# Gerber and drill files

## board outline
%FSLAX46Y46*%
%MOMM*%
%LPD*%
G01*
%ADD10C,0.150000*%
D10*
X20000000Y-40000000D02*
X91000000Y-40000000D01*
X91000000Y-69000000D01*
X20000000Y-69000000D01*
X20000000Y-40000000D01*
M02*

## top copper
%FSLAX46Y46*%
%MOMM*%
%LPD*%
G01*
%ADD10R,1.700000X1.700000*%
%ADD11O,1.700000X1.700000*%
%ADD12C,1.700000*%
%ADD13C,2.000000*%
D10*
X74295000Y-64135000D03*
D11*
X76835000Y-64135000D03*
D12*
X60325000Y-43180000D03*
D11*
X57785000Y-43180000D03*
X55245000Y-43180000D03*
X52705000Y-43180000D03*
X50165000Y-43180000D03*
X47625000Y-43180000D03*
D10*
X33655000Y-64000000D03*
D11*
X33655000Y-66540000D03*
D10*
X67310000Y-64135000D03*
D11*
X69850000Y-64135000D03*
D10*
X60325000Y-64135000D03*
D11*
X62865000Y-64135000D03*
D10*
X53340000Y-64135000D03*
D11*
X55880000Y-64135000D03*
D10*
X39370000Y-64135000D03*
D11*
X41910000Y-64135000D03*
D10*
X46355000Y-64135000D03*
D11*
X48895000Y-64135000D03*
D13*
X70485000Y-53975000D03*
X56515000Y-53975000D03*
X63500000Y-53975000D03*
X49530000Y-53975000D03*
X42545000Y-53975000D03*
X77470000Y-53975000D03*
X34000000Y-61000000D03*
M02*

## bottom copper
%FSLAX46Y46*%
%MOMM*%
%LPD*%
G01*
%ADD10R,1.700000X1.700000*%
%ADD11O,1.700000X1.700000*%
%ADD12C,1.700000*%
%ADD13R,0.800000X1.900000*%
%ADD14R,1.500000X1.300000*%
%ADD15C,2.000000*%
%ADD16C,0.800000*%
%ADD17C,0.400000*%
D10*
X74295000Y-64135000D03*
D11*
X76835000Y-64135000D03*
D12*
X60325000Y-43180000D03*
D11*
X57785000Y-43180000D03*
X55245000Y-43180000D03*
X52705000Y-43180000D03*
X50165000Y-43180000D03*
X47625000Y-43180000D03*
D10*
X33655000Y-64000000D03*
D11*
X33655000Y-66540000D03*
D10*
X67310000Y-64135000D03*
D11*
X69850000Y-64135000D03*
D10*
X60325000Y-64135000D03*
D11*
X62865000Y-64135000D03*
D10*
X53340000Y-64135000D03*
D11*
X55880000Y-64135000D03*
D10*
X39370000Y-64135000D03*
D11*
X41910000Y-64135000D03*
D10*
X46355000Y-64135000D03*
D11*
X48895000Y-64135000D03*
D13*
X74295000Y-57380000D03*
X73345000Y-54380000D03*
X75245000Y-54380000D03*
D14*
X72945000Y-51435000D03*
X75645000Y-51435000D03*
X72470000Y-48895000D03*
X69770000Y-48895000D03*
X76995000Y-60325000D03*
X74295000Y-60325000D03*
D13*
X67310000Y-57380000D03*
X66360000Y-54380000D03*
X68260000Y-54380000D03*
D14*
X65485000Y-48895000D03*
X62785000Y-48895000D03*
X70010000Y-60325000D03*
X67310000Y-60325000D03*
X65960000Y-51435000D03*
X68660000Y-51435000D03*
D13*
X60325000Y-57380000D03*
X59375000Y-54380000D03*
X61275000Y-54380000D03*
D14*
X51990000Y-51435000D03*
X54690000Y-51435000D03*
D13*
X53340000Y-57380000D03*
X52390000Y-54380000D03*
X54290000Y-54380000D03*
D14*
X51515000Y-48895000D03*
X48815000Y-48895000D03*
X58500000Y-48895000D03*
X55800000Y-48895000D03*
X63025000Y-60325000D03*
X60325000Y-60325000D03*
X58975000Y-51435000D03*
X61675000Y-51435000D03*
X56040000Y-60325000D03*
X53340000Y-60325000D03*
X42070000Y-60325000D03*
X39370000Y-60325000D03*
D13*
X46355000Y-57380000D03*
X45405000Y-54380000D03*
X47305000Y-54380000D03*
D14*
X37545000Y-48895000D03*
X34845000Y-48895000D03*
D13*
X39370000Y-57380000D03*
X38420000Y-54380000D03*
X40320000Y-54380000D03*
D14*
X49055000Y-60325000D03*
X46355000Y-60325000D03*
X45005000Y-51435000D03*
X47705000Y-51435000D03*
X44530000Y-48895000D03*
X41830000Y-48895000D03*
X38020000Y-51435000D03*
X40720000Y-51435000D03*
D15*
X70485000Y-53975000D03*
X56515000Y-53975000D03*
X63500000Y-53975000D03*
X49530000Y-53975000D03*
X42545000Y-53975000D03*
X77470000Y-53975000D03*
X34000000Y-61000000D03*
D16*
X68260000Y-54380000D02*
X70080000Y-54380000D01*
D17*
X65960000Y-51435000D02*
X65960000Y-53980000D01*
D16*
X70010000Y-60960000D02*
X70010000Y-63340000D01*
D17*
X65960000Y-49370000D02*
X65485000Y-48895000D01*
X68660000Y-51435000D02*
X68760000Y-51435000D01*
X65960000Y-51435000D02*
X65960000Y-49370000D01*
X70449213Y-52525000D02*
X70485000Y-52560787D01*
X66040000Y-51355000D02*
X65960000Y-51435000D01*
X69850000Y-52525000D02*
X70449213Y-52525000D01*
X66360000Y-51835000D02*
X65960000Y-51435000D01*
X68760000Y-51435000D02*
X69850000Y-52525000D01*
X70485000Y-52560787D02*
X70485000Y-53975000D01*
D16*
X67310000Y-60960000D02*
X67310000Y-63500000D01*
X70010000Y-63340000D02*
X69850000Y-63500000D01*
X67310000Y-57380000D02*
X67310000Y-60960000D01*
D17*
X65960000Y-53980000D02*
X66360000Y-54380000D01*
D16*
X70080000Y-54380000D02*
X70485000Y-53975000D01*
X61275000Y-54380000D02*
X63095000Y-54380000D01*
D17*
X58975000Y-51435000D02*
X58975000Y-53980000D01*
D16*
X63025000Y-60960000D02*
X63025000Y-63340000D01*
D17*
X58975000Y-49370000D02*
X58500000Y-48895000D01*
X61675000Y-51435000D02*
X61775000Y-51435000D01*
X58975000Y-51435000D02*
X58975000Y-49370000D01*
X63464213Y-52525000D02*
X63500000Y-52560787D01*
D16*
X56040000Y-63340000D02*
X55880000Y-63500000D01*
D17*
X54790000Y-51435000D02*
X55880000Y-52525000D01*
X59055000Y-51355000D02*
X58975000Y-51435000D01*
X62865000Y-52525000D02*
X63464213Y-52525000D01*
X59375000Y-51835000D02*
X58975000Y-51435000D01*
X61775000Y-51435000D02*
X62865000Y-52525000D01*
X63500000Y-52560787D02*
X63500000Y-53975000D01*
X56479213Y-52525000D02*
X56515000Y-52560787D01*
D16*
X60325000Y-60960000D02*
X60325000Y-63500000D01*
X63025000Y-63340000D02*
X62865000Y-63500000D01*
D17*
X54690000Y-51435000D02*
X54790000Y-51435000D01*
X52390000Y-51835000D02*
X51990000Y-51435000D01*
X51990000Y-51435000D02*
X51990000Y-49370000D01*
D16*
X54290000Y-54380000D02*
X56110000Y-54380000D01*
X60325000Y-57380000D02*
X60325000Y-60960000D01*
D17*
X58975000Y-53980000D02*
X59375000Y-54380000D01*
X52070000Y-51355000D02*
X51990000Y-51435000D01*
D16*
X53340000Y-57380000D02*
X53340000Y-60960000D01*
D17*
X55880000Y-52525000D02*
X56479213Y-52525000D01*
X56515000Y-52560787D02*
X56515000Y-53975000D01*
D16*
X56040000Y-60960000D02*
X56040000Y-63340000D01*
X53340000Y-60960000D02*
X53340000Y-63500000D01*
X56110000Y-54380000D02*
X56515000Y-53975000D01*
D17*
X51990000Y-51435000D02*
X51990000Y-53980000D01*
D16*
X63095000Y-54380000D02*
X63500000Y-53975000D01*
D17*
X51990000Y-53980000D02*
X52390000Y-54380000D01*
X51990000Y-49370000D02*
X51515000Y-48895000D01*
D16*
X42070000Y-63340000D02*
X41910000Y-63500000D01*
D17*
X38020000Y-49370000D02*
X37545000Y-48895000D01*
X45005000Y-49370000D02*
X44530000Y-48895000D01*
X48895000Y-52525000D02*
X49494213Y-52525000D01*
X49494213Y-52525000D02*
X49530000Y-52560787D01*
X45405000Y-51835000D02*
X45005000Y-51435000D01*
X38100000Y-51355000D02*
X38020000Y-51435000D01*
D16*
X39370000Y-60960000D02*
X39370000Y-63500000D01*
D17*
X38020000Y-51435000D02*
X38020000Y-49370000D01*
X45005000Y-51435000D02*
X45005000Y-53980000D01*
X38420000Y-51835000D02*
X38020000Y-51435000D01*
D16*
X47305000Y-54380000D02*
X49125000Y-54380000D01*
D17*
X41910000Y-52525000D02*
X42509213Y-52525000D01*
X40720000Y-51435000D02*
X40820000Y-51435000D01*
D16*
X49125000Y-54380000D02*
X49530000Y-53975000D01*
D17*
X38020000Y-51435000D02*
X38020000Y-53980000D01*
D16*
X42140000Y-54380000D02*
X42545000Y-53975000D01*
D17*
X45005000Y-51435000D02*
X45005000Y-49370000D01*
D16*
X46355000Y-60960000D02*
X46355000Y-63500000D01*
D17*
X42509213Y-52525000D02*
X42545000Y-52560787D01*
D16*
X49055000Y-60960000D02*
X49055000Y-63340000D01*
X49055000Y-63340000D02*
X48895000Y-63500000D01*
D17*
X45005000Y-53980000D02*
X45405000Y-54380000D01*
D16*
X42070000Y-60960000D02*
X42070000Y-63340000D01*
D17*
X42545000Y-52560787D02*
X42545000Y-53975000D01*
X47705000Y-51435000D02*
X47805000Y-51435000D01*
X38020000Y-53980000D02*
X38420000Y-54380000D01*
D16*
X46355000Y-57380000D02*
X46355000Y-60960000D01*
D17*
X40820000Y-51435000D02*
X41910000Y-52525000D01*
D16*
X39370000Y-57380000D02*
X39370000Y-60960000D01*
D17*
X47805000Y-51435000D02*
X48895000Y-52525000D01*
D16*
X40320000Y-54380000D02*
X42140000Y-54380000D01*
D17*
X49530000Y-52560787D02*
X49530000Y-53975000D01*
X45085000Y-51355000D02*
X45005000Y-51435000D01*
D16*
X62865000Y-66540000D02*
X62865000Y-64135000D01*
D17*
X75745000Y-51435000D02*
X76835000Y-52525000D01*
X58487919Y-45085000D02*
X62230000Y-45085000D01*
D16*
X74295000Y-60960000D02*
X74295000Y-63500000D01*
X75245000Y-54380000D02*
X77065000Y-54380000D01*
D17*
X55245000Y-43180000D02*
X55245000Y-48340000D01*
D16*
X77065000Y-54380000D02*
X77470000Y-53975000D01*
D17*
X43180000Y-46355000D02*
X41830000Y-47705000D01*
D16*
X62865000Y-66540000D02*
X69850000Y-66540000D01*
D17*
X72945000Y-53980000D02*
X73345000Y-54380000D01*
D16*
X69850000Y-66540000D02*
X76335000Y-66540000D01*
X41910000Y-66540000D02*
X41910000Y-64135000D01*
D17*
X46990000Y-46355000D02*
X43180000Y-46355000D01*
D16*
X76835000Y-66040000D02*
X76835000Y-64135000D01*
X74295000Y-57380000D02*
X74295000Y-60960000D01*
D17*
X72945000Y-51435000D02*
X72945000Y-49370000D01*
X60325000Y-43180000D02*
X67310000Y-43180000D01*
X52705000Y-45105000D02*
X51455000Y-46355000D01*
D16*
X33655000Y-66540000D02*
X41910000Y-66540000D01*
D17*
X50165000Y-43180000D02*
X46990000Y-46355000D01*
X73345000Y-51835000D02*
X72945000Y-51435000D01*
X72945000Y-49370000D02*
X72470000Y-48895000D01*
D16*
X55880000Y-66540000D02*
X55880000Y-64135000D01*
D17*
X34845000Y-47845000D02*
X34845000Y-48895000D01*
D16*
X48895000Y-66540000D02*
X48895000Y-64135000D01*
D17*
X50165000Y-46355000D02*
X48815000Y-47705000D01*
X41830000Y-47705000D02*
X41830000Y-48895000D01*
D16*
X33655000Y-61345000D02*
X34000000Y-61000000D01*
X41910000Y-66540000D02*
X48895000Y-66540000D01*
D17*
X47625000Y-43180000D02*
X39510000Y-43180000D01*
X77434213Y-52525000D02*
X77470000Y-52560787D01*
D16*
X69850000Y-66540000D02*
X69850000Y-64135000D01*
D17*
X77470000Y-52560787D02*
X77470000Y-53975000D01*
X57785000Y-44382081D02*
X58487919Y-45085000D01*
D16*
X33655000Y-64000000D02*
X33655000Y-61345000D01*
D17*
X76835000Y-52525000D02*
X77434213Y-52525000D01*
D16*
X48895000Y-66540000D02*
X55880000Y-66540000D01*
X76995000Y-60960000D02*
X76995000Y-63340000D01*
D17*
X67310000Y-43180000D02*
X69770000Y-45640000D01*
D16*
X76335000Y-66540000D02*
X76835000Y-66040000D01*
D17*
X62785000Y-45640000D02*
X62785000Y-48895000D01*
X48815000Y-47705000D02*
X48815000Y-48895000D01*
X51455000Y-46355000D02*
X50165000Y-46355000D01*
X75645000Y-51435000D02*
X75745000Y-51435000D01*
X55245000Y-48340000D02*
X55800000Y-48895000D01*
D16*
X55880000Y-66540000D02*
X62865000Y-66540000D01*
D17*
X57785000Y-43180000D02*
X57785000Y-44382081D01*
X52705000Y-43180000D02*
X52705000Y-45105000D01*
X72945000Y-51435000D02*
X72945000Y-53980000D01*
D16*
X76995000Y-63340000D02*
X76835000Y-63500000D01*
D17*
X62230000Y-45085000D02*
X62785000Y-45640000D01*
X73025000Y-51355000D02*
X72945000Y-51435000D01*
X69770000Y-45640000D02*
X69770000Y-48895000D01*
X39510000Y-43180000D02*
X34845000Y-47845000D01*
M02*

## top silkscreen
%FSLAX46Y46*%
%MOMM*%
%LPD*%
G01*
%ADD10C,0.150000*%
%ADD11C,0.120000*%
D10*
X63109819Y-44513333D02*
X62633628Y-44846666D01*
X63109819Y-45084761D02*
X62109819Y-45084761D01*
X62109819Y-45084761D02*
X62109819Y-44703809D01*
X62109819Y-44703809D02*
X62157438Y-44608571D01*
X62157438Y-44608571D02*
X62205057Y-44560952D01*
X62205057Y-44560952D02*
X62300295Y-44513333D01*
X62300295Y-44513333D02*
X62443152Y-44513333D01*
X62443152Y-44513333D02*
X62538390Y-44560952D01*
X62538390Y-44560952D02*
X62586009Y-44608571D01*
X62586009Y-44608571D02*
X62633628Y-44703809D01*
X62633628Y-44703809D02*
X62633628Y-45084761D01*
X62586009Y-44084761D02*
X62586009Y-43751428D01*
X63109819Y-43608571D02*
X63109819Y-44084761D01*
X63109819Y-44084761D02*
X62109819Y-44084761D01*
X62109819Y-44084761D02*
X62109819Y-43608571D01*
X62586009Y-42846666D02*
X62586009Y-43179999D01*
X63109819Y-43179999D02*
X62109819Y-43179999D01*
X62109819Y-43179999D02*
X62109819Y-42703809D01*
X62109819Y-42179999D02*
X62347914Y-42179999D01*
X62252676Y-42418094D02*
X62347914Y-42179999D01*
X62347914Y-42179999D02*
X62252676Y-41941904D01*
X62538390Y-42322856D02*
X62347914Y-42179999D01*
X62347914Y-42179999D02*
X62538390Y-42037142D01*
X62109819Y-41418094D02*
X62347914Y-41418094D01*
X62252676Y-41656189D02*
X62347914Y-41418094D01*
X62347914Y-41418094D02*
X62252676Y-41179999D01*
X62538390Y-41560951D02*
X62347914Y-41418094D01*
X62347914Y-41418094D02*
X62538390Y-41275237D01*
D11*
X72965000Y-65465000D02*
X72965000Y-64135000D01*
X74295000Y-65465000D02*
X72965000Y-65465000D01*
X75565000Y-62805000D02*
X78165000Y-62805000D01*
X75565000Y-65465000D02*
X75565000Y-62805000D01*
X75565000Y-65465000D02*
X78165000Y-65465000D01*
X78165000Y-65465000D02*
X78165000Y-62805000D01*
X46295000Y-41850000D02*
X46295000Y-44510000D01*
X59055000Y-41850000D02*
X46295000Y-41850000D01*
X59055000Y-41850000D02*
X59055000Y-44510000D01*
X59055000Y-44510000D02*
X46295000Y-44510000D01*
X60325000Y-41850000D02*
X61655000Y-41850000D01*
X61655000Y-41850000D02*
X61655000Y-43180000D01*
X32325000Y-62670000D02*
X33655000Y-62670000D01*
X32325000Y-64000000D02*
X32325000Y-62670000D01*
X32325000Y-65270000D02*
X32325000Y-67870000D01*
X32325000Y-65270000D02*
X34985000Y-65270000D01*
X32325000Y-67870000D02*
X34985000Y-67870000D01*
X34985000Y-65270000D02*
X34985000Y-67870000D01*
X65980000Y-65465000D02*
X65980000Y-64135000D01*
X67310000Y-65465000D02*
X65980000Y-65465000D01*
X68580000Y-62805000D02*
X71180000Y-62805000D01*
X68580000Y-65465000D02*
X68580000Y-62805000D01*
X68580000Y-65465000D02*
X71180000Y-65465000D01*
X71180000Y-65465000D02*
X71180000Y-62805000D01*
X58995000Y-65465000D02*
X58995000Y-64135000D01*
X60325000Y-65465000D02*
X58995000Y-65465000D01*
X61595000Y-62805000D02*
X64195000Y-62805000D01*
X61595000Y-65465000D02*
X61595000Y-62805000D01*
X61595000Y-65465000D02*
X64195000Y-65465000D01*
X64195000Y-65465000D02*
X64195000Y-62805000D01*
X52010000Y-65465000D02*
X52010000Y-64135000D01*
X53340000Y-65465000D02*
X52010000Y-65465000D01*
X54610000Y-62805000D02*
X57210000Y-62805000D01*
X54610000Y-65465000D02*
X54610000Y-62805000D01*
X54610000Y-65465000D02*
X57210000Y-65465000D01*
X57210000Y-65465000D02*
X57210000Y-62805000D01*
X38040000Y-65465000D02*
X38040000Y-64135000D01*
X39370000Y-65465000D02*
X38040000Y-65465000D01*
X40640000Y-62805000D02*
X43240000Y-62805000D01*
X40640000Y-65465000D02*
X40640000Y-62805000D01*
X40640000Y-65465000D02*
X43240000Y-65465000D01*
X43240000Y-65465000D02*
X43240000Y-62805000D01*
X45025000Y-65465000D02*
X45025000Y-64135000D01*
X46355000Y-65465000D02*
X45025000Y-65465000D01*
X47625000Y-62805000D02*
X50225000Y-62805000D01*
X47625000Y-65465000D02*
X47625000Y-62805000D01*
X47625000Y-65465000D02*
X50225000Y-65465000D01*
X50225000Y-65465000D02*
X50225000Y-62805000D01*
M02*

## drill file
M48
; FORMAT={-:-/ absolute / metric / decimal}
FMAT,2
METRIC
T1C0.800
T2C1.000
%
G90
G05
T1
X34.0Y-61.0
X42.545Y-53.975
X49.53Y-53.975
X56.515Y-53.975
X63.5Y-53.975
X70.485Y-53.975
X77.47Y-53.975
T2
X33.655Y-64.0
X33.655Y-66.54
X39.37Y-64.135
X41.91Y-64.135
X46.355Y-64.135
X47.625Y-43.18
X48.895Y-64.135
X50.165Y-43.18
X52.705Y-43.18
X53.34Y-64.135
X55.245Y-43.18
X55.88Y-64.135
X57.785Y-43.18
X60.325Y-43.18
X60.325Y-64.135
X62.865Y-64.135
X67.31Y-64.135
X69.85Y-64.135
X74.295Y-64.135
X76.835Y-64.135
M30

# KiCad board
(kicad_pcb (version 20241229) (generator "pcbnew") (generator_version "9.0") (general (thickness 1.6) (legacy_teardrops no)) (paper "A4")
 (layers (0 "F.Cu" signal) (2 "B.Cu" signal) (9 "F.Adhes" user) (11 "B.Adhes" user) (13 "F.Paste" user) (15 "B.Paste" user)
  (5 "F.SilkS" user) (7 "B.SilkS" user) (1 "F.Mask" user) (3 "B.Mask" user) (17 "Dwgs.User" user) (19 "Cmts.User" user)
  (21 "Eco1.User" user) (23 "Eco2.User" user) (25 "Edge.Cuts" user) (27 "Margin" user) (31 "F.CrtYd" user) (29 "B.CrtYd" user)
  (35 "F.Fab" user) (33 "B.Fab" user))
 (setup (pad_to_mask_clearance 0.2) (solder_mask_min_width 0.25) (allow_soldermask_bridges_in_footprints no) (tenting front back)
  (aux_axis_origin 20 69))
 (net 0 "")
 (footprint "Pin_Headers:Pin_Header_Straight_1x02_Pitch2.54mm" (layer "F.Cu") (at 74.295 64.135 90)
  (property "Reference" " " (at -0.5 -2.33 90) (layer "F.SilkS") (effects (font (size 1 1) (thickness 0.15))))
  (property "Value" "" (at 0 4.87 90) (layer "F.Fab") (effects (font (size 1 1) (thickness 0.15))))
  (fp_line (start -1.33 -1.33) (end 0 -1.33) (stroke (width 0.12) (type solid)) (layer "F.SilkS"))
  (fp_line (start -1.33 0) (end -1.33 -1.33) (stroke (width 0.12) (type solid)) (layer "F.SilkS"))
  (fp_line (start 1.33 1.27) (end 1.33 3.87) (stroke (width 0.12) (type solid)) (layer "F.SilkS"))
  (fp_line (start -1.33 1.27) (end 1.33 1.27) (stroke (width 0.12) (type solid)) (layer "F.SilkS"))
  (fp_line (start -1.33 1.27) (end -1.33 3.87) (stroke (width 0.12) (type solid)) (layer "F.SilkS"))
  (fp_line (start -1.33 3.87) (end 1.33 3.87) (stroke (width 0.12) (type solid)) (layer "F.SilkS"))
  (pad "1" thru_hole rect (at 0 0 90) (size 1.7 1.7) (drill 1) (layers "*.Cu" "*.Mask") (remove_unused_layers no))
  (pad "2" thru_hole oval (at 0 2.54 90) (size 1.7 1.7) (drill 1) (layers "*.Cu" "*.Mask") (remove_unused_layers no)))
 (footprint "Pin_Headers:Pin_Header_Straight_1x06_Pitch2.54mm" (layer "F.Cu") (at 60.325 43.18 -90)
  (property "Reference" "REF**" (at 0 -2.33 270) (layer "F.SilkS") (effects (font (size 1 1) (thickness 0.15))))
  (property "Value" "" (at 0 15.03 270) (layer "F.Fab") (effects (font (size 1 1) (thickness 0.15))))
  (fp_line (start -1.33 14.03) (end 1.33 14.03) (stroke (width 0.12) (type solid)) (layer "F.SilkS"))
  (fp_line (start -1.33 1.27) (end -1.33 14.03) (stroke (width 0.12) (type solid)) (layer "F.SilkS"))
  (fp_line (start -1.33 1.27) (end 1.33 1.27) (stroke (width 0.12) (type solid)) (layer "F.SilkS"))
  (fp_line (start 1.33 1.27) (end 1.33 14.03) (stroke (width 0.12) (type solid)) (layer "F.SilkS"))
  (fp_line (start -1.33 0) (end -1.33 -1.33) (stroke (width 0.12) (type solid)) (layer "F.SilkS"))
  (fp_line (start -1.33 -1.33) (end 0 -1.33) (stroke (width 0.12) (type solid)) (layer "F.SilkS"))
  (pad "1" thru_hole circle (at 0 0 270) (size 1.7 1.7) (drill 1) (layers "*.Cu" "*.Mask") (remove_unused_layers no))
  (pad "2" thru_hole oval (at 0 2.54 270) (size 1.7 1.7) (drill 1) (layers "*.Cu" "*.Mask") (remove_unused_layers no))
  (pad "3" thru_hole oval (at 0 5.08 270) (size 1.7 1.7) (drill 1) (layers "*.Cu" "*.Mask") (remove_unused_layers no))
  (pad "4" thru_hole oval (at 0 7.62 270) (size 1.7 1.7) (drill 1) (layers "*.Cu" "*.Mask") (remove_unused_layers no))
  (pad "5" thru_hole oval (at 0 10.16 270) (size 1.7 1.7) (drill 1) (layers "*.Cu" "*.Mask") (remove_unused_layers no))
  (pad "6" thru_hole oval (at 0 12.7 270) (size 1.7 1.7) (drill 1) (layers "*.Cu" "*.Mask") (remove_unused_layers no)))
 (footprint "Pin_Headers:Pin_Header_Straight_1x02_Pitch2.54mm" (layer "F.Cu") (at 33.655 64)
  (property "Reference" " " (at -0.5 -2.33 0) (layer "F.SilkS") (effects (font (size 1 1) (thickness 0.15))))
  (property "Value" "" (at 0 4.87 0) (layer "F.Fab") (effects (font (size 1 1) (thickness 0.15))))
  (fp_line (start -1.33 -1.33) (end 0 -1.33) (stroke (width 0.12) (type solid)) (layer "F.SilkS"))
  (fp_line (start -1.33 0) (end -1.33 -1.33) (stroke (width 0.12) (type solid)) (layer "F.SilkS"))
  (fp_line (start -1.33 1.27) (end -1.33 3.87) (stroke (width 0.12) (type solid)) (layer "F.SilkS"))
  (fp_line (start -1.33 1.27) (end 1.33 1.27) (stroke (width 0.12) (type solid)) (layer "F.SilkS"))
  (fp_line (start -1.33 3.87) (end 1.33 3.87) (stroke (width 0.12) (type solid)) (layer "F.SilkS"))
  (fp_line (start 1.33 1.27) (end 1.33 3.87) (stroke (width 0.12) (type solid)) (layer "F.SilkS"))
  (pad "1" thru_hole rect (at 0 0) (size 1.7 1.7) (drill 1) (layers "*.Cu" "*.Mask") (remove_unused_layers no))
  (pad "2" thru_hole oval (at 0 2.54) (size 1.7 1.7) (drill 1) (layers "*.Cu" "*.Mask") (remove_unused_layers no)))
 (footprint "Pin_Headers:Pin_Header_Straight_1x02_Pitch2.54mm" (layer "F.Cu") (at 67.31 64.135 90)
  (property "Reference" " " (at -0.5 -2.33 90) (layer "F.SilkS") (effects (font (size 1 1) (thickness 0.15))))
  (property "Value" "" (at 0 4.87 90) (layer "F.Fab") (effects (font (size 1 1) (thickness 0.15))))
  (fp_line (start -1.33 -1.33) (end 0 -1.33) (stroke (width 0.12) (type solid)) (layer "F.SilkS"))
  (fp_line (start -1.33 0) (end -1.33 -1.33) (stroke (width 0.12) (type solid)) (layer "F.SilkS"))
  (fp_line (start 1.33 1.27) (end 1.33 3.87) (stroke (width 0.12) (type solid)) (layer "F.SilkS"))
  (fp_line (start -1.33 1.27) (end 1.33 1.27) (stroke (width 0.12) (type solid)) (layer "F.SilkS"))
  (fp_line (start -1.33 1.27) (end -1.33 3.87) (stroke (width 0.12) (type solid)) (layer "F.SilkS"))
  (fp_line (start -1.33 3.87) (end 1.33 3.87) (stroke (width 0.12) (type solid)) (layer "F.SilkS"))
  (pad "1" thru_hole rect (at 0 0 90) (size 1.7 1.7) (drill 1) (layers "*.Cu" "*.Mask") (remove_unused_layers no))
  (pad "2" thru_hole oval (at 0 2.54 90) (size 1.7 1.7) (drill 1) (layers "*.Cu" "*.Mask") (remove_unused_layers no)))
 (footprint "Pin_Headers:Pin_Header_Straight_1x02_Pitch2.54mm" (layer "F.Cu") (at 60.325 64.135 90)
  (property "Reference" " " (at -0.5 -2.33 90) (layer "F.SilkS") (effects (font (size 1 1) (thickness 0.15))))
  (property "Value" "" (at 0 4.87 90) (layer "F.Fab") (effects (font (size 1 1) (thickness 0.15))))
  (fp_line (start -1.33 -1.33) (end 0 -1.33) (stroke (width 0.12) (type solid)) (layer "F.SilkS"))
  (fp_line (start -1.33 0) (end -1.33 -1.33) (stroke (width 0.12) (type solid)) (layer "F.SilkS"))
  (fp_line (start 1.33 1.27) (end 1.33 3.87) (stroke (width 0.12) (type solid)) (layer "F.SilkS"))
  (fp_line (start -1.33 1.27) (end 1.33 1.27) (stroke (width 0.12) (type solid)) (layer "F.SilkS"))
  (fp_line (start -1.33 1.27) (end -1.33 3.87) (stroke (width 0.12) (type solid)) (layer "F.SilkS"))
  (fp_line (start -1.33 3.87) (end 1.33 3.87) (stroke (width 0.12) (type solid)) (layer "F.SilkS"))
  (pad "1" thru_hole rect (at 0 0 90) (size 1.7 1.7) (drill 1) (layers "*.Cu" "*.Mask") (remove_unused_layers no))
  (pad "2" thru_hole oval (at 0 2.54 90) (size 1.7 1.7) (drill 1) (layers "*.Cu" "*.Mask") (remove_unused_layers no)))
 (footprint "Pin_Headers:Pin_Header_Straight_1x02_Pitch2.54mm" (layer "F.Cu") (at 53.34 64.135 90)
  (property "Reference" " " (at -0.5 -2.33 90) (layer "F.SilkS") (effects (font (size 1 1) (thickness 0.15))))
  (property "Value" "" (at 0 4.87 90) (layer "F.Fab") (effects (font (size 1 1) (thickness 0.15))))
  (fp_line (start -1.33 -1.33) (end 0 -1.33) (stroke (width 0.12) (type solid)) (layer "F.SilkS"))
  (fp_line (start -1.33 0) (end -1.33 -1.33) (stroke (width 0.12) (type solid)) (layer "F.SilkS"))
  (fp_line (start 1.33 1.27) (end 1.33 3.87) (stroke (width 0.12) (type solid)) (layer "F.SilkS"))
  (fp_line (start -1.33 1.27) (end 1.33 1.27) (stroke (width 0.12) (type solid)) (layer "F.SilkS"))
  (fp_line (start -1.33 1.27) (end -1.33 3.87) (stroke (width 0.12) (type solid)) (layer "F.SilkS"))
  (fp_line (start -1.33 3.87) (end 1.33 3.87) (stroke (width 0.12) (type solid)) (layer "F.SilkS"))
  (pad "1" thru_hole rect (at 0 0 90) (size 1.7 1.7) (drill 1) (layers "*.Cu" "*.Mask") (remove_unused_layers no))
  (pad "2" thru_hole oval (at 0 2.54 90) (size 1.7 1.7) (drill 1) (layers "*.Cu" "*.Mask") (remove_unused_layers no)))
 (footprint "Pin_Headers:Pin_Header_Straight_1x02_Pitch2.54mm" (layer "F.Cu") (at 39.37 64.135 90)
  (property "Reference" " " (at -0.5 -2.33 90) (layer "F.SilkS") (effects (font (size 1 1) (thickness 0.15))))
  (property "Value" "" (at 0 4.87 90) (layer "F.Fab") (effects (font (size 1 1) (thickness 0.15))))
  (fp_line (start -1.33 -1.33) (end 0 -1.33) (stroke (width 0.12) (type solid)) (layer "F.SilkS"))
  (fp_line (start -1.33 0) (end -1.33 -1.33) (stroke (width 0.12) (type solid)) (layer "F.SilkS"))
  (fp_line (start 1.33 1.27) (end 1.33 3.87) (stroke (width 0.12) (type solid)) (layer "F.SilkS"))
  (fp_line (start -1.33 1.27) (end 1.33 1.27) (stroke (width 0.12) (type solid)) (layer "F.SilkS"))
  (fp_line (start -1.33 1.27) (end -1.33 3.87) (stroke (width 0.12) (type solid)) (layer "F.SilkS"))
  (fp_line (start -1.33 3.87) (end 1.33 3.87) (stroke (width 0.12) (type solid)) (layer "F.SilkS"))
  (pad "1" thru_hole rect (at 0 0 90) (size 1.7 1.7) (drill 1) (layers "*.Cu" "*.Mask") (remove_unused_layers no))
  (pad "2" thru_hole oval (at 0 2.54 90) (size 1.7 1.7) (drill 1) (layers "*.Cu" "*.Mask") (remove_unused_layers no)))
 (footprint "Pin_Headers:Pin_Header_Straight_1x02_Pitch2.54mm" (layer "F.Cu") (at 46.355 64.135 90)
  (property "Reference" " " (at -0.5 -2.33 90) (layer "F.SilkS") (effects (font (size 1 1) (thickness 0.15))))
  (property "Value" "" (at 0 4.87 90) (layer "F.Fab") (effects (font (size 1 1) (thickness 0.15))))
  (fp_line (start -1.33 -1.33) (end 0 -1.33) (stroke (width 0.12) (type solid)) (layer "F.SilkS"))
  (fp_line (start -1.33 0) (end -1.33 -1.33) (stroke (width 0.12) (type solid)) (layer "F.SilkS"))
  (fp_line (start 1.33 1.27) (end 1.33 3.87) (stroke (width 0.12) (type solid)) (layer "F.SilkS"))
  (fp_line (start -1.33 1.27) (end 1.33 1.27) (stroke (width 0.12) (type solid)) (layer "F.SilkS"))
  (fp_line (start -1.33 1.27) (end -1.33 3.87) (stroke (width 0.12) (type solid)) (layer "F.SilkS"))
  (fp_line (start -1.33 3.87) (end 1.33 3.87) (stroke (width 0.12) (type solid)) (layer "F.SilkS"))
  (pad "1" thru_hole rect (at 0 0 90) (size 1.7 1.7) (drill 1) (layers "*.Cu" "*.Mask") (remove_unused_layers no))
  (pad "2" thru_hole oval (at 0 2.54 90) (size 1.7 1.7) (drill 1) (layers "*.Cu" "*.Mask") (remove_unused_layers no)))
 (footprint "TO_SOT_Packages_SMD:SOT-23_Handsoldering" (layer "B.Cu") (at 74.295 55.88 -90)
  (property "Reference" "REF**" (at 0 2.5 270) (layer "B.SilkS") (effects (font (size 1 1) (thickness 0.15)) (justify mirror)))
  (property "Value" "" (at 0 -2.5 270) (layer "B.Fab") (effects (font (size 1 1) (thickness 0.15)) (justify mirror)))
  (pad "D" smd rect (at 1.5 0 270) (size 1.9 0.8) (layers "B.Cu" "B.Mask" "B.Paste"))
  (pad "G" smd rect (at -1.5 0.95 270) (size 1.9 0.8) (layers "B.Cu" "B.Mask" "B.Paste"))
  (pad "S" smd rect (at -1.5 -0.95 270) (size 1.9 0.8) (layers "B.Cu" "B.Mask" "B.Paste")))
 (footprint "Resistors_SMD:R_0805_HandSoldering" (layer "B.Cu") (at 74.295 51.435)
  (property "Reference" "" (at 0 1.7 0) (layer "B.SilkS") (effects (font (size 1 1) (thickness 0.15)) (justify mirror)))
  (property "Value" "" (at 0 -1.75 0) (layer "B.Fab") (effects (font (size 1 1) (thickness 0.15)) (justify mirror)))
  (pad "1" smd rect (at -1.35 0) (size 1.5 1.3) (layers "B.Cu" "B.Mask" "B.Paste"))
  (pad "2" smd rect (at 1.35 0) (size 1.5 1.3) (layers "B.Cu" "B.Mask" "B.Paste")))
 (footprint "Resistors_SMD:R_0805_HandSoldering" (layer "B.Cu") (at 71.12 48.895 180)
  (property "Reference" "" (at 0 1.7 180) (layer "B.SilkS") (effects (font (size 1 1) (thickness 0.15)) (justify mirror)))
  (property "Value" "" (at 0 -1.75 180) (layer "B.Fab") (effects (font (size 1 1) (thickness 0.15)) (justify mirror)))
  (pad "1" smd rect (at -1.35 0 180) (size 1.5 1.3) (layers "B.Cu" "B.Mask" "B.Paste"))
  (pad "2" smd rect (at 1.35 0 180) (size 1.5 1.3) (layers "B.Cu" "B.Mask" "B.Paste")))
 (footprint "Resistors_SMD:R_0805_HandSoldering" (layer "B.Cu") (at 75.645 60.325 180)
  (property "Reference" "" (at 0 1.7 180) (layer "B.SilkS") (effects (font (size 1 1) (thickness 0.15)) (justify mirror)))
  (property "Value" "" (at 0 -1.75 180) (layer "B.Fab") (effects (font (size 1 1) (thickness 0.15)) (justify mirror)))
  (pad "1" smd rect (at -1.35 0 180) (size 1.5 1.3) (layers "B.Cu" "B.Mask" "B.Paste"))
  (pad "2" smd rect (at 1.35 0 180) (size 1.5 1.3) (layers "B.Cu" "B.Mask" "B.Paste")))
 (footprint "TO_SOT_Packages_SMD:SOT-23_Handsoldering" (layer "B.Cu") (at 67.31 55.88 -90)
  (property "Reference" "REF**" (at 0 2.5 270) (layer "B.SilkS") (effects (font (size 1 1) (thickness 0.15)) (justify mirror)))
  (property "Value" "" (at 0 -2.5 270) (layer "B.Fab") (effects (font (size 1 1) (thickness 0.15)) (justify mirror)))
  (pad "D" smd rect (at 1.5 0 270) (size 1.9 0.8) (layers "B.Cu" "B.Mask" "B.Paste"))
  (pad "G" smd rect (at -1.5 0.95 270) (size 1.9 0.8) (layers "B.Cu" "B.Mask" "B.Paste"))
  (pad "S" smd rect (at -1.5 -0.95 270) (size 1.9 0.8) (layers "B.Cu" "B.Mask" "B.Paste")))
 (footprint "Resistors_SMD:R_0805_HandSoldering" (layer "B.Cu") (at 64.135 48.895 180)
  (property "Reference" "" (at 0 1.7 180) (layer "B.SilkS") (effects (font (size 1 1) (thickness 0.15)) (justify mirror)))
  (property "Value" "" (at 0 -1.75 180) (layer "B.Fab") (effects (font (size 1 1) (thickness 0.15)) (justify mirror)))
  (pad "1" smd rect (at -1.35 0 180) (size 1.5 1.3) (layers "B.Cu" "B.Mask" "B.Paste"))
  (pad "2" smd rect (at 1.35 0 180) (size 1.5 1.3) (layers "B.Cu" "B.Mask" "B.Paste")))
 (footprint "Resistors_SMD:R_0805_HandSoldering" (layer "B.Cu") (at 68.66 60.325 180)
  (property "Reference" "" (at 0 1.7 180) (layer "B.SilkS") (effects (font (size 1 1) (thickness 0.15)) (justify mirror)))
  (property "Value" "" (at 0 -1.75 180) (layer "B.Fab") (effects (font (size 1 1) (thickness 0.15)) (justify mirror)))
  (pad "1" smd rect (at -1.35 0 180) (size 1.5 1.3) (layers "B.Cu" "B.Mask" "B.Paste"))
  (pad "2" smd rect (at 1.35 0 180) (size 1.5 1.3) (layers "B.Cu" "B.Mask" "B.Paste")))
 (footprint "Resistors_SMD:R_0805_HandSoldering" (layer "B.Cu") (at 67.31 51.435)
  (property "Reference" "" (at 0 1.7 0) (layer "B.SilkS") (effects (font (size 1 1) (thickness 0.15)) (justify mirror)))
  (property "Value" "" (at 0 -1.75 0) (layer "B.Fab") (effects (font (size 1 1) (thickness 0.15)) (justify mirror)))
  (pad "1" smd rect (at -1.35 0) (size 1.5 1.3) (layers "B.Cu" "B.Mask" "B.Paste"))
  (pad "2" smd rect (at 1.35 0) (size 1.5 1.3) (layers "B.Cu" "B.Mask" "B.Paste")))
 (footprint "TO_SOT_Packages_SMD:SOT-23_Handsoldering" (layer "B.Cu") (at 60.325 55.88 -90)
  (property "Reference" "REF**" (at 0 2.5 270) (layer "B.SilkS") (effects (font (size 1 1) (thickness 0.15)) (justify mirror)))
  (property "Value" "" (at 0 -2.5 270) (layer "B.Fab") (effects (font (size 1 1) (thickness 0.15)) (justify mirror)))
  (pad "D" smd rect (at 1.5 0 270) (size 1.9 0.8) (layers "B.Cu" "B.Mask" "B.Paste"))
  (pad "G" smd rect (at -1.5 0.95 270) (size 1.9 0.8) (layers "B.Cu" "B.Mask" "B.Paste"))
  (pad "S" smd rect (at -1.5 -0.95 270) (size 1.9 0.8) (layers "B.Cu" "B.Mask" "B.Paste")))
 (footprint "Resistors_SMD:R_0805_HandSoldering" (layer "B.Cu") (at 53.34 51.435)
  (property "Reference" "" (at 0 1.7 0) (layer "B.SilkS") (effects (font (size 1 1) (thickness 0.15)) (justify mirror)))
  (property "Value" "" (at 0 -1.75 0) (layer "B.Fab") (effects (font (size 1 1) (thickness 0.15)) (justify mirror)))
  (pad "1" smd rect (at -1.35 0) (size 1.5 1.3) (layers "B.Cu" "B.Mask" "B.Paste"))
  (pad "2" smd rect (at 1.35 0) (size 1.5 1.3) (layers "B.Cu" "B.Mask" "B.Paste")))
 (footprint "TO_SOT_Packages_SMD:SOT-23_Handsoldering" (layer "B.Cu") (at 53.34 55.88 -90)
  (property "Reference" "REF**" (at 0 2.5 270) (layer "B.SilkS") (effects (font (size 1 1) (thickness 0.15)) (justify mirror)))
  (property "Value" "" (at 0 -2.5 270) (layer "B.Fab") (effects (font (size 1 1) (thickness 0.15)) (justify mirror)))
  (pad "D" smd rect (at 1.5 0 270) (size 1.9 0.8) (layers "B.Cu" "B.Mask" "B.Paste"))
  (pad "G" smd rect (at -1.5 0.95 270) (size 1.9 0.8) (layers "B.Cu" "B.Mask" "B.Paste"))
  (pad "S" smd rect (at -1.5 -0.95 270) (size 1.9 0.8) (layers "B.Cu" "B.Mask" "B.Paste")))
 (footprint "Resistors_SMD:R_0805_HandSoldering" (layer "B.Cu") (at 50.165 48.895 180)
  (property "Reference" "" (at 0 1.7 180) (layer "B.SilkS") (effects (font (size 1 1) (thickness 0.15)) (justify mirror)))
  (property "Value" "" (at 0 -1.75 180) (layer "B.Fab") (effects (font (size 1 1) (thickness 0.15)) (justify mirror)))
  (pad "1" smd rect (at -1.35 0 180) (size 1.5 1.3) (layers "B.Cu" "B.Mask" "B.Paste"))
  (pad "2" smd rect (at 1.35 0 180) (size 1.5 1.3) (layers "B.Cu" "B.Mask" "B.Paste")))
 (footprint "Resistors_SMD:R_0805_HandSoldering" (layer "B.Cu") (at 57.15 48.895 180)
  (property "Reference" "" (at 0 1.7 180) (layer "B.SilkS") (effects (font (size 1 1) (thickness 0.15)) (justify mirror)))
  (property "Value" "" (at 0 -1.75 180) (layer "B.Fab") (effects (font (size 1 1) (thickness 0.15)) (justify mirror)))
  (pad "1" smd rect (at -1.35 0 180) (size 1.5 1.3) (layers "B.Cu" "B.Mask" "B.Paste"))
  (pad "2" smd rect (at 1.35 0 180) (size 1.5 1.3) (layers "B.Cu" "B.Mask" "B.Paste")))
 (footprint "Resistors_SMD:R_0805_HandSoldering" (layer "B.Cu") (at 61.675 60.325 180)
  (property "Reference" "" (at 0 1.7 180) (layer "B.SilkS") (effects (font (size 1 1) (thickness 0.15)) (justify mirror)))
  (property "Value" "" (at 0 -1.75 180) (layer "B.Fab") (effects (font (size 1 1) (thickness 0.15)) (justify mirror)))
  (pad "1" smd rect (at -1.35 0 180) (size 1.5 1.3) (layers "B.Cu" "B.Mask" "B.Paste"))
  (pad "2" smd rect (at 1.35 0 180) (size 1.5 1.3) (layers "B.Cu" "B.Mask" "B.Paste")))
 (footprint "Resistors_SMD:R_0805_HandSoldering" (layer "B.Cu") (at 60.325 51.435)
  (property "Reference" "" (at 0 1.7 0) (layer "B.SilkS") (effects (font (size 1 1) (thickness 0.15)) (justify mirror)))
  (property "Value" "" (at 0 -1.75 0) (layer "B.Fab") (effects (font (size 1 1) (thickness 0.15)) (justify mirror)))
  (pad "1" smd rect (at -1.35 0) (size 1.5 1.3) (layers "B.Cu" "B.Mask" "B.Paste"))
  (pad "2" smd rect (at 1.35 0) (size 1.5 1.3) (layers "B.Cu" "B.Mask" "B.Paste")))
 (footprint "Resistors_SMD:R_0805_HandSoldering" (layer "B.Cu") (at 54.69 60.325 180)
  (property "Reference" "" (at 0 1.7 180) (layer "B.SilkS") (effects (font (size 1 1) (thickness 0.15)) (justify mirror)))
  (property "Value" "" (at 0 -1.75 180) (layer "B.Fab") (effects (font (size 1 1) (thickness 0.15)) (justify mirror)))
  (pad "1" smd rect (at -1.35 0 180) (size 1.5 1.3) (layers "B.Cu" "B.Mask" "B.Paste"))
  (pad "2" smd rect (at 1.35 0 180) (size 1.5 1.3) (layers "B.Cu" "B.Mask" "B.Paste")))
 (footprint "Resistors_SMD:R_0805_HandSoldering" (layer "B.Cu") (at 40.72 60.325 180)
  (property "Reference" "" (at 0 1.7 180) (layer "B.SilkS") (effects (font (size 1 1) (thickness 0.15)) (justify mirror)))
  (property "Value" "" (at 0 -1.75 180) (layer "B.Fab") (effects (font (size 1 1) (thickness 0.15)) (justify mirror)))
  (pad "1" smd rect (at -1.35 0 180) (size 1.5 1.3) (layers "B.Cu" "B.Mask" "B.Paste"))
  (pad "2" smd rect (at 1.35 0 180) (size 1.5 1.3) (layers "B.Cu" "B.Mask" "B.Paste")))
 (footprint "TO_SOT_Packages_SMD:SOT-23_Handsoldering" (layer "B.Cu") (at 46.355 55.88 -90)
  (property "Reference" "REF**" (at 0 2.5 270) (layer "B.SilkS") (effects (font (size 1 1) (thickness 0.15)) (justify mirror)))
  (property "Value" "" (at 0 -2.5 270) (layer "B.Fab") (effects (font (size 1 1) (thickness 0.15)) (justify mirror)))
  (pad "D" smd rect (at 1.5 0 270) (size 1.9 0.8) (layers "B.Cu" "B.Mask" "B.Paste"))
  (pad "G" smd rect (at -1.5 0.95 270) (size 1.9 0.8) (layers "B.Cu" "B.Mask" "B.Paste"))
  (pad "S" smd rect (at -1.5 -0.95 270) (size 1.9 0.8) (layers "B.Cu" "B.Mask" "B.Paste")))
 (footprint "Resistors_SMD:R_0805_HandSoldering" (layer "B.Cu") (at 36.195 48.895 180)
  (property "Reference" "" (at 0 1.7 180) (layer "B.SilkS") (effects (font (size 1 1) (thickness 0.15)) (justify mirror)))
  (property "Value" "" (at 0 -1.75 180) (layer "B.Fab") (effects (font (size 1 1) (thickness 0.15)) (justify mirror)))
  (pad "1" smd rect (at -1.35 0 180) (size 1.5 1.3) (layers "B.Cu" "B.Mask" "B.Paste"))
  (pad "2" smd rect (at 1.35 0 180) (size 1.5 1.3) (layers "B.Cu" "B.Mask" "B.Paste")))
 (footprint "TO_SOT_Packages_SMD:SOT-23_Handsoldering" (layer "B.Cu") (at 39.37 55.88 -90)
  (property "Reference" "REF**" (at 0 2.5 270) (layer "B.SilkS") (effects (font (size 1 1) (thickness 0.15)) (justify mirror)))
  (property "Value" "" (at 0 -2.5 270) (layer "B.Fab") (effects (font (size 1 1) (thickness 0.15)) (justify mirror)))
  (pad "D" smd rect (at 1.5 0 270) (size 1.9 0.8) (layers "B.Cu" "B.Mask" "B.Paste"))
  (pad "G" smd rect (at -1.5 0.95 270) (size 1.9 0.8) (layers "B.Cu" "B.Mask" "B.Paste"))
  (pad "S" smd rect (at -1.5 -0.95 270) (size 1.9 0.8) (layers "B.Cu" "B.Mask" "B.Paste")))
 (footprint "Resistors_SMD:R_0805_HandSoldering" (layer "B.Cu") (at 47.705 60.325 180)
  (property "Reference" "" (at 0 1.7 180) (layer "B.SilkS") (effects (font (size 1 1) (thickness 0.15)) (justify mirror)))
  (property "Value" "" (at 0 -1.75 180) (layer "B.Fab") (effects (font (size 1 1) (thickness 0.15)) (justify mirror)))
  (pad "1" smd rect (at -1.35 0 180) (size 1.5 1.3) (layers "B.Cu" "B.Mask" "B.Paste"))
  (pad "2" smd rect (at 1.35 0 180) (size 1.5 1.3) (layers "B.Cu" "B.Mask" "B.Paste")))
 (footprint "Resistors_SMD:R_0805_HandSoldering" (layer "B.Cu") (at 46.355 51.435)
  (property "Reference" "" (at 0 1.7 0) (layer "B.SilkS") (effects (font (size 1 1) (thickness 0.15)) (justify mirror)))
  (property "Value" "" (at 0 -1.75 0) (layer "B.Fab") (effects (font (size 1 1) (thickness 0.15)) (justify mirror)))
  (pad "1" smd rect (at -1.35 0) (size 1.5 1.3) (layers "B.Cu" "B.Mask" "B.Paste"))
  (pad "2" smd rect (at 1.35 0) (size 1.5 1.3) (layers "B.Cu" "B.Mask" "B.Paste")))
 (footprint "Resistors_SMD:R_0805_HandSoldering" (layer "B.Cu") (at 43.18 48.895 180)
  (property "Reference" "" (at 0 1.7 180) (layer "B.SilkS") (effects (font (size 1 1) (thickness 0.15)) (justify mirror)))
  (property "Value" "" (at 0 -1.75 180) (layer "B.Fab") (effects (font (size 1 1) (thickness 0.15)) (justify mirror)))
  (pad "1" smd rect (at -1.35 0 180) (size 1.5 1.3) (layers "B.Cu" "B.Mask" "B.Paste"))
  (pad "2" smd rect (at 1.35 0 180) (size 1.5 1.3) (layers "B.Cu" "B.Mask" "B.Paste")))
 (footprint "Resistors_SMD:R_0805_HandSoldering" (layer "B.Cu") (at 39.37 51.435)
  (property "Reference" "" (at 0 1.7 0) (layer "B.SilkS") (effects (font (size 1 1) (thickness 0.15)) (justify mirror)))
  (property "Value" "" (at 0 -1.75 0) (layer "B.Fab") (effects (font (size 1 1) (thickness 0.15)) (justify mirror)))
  (pad "1" smd rect (at -1.35 0) (size 1.5 1.3) (layers "B.Cu" "B.Mask" "B.Paste"))
  (pad "2" smd rect (at 1.35 0) (size 1.5 1.3) (layers "B.Cu" "B.Mask" "B.Paste")))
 (gr_poly (pts (xy 20 40) (xy 91 40) (xy 91 69) (xy 20 69)) (stroke (width 0.15) (type solid)) (fill no) (layer "Edge.Cuts"))
 (via (at 70.485 53.975) (size 2) (drill 0.8) (layers "F.Cu" "B.Cu") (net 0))
 (via (at 56.515 53.975) (size 2) (drill 0.8) (layers "F.Cu" "B.Cu") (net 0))
 (via (at 63.5 53.975) (size 2) (drill 0.8) (layers "F.Cu" "B.Cu") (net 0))
 (via (at 49.53 53.975) (size 2) (drill 0.8) (layers "F.Cu" "B.Cu") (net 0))
 (via (at 42.545 53.975) (size 2) (drill 0.8) (layers "F.Cu" "B.Cu") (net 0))
 (via (at 77.47 53.975) (size 2) (drill 0.8) (layers "F.Cu" "B.Cu") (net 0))
 (via (at 34 61) (size 2) (drill 0.8) (layers "F.Cu" "B.Cu") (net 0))
 (segment (start 68.26 54.38) (end 70.08 54.38) (width 0.8) (layer "B.Cu") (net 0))
 (segment (start 65.96 51.435) (end 65.96 53.98) (width 0.4) (layer "B.Cu") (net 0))
 (segment (start 70.01 60.96) (end 70.01 63.34) (width 0.8) (layer "B.Cu") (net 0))
 (segment (start 65.96 49.37) (end 65.485 48.895) (width 0.4) (layer "B.Cu") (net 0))
 (segment (start 68.66 51.435) (end 68.76 51.435) (width 0.4) (layer "B.Cu") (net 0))
 (segment (start 65.96 51.435) (end 65.96 49.37) (width 0.4) (layer "B.Cu") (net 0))
 (segment (start 70.449213 52.525) (end 70.485 52.560787) (width 0.4) (layer "B.Cu") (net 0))
 (segment (start 66.04 51.355) (end 65.96 51.435) (width 0.4) (layer "B.Cu") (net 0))
 (segment (start 69.85 52.525) (end 70.449213 52.525) (width 0.4) (layer "B.Cu") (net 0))
 (segment (start 66.36 51.835) (end 65.96 51.435) (width 0.4) (layer "B.Cu") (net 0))
 (segment (start 68.76 51.435) (end 69.85 52.525) (width 0.4) (layer "B.Cu") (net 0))
 (segment (start 70.485 52.560787) (end 70.485 53.975) (width 0.4) (layer "B.Cu") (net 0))
 (segment (start 67.31 60.96) (end 67.31 63.5) (width 0.8) (layer "B.Cu") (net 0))
 (segment (start 70.01 63.34) (end 69.85 63.5) (width 0.8) (layer "B.Cu") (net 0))
 (segment (start 67.31 57.38) (end 67.31 60.96) (width 0.8) (layer "B.Cu") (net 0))
 (segment (start 65.96 53.98) (end 66.36 54.38) (width 0.4) (layer "B.Cu") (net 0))
 (segment (start 70.08 54.38) (end 70.485 53.975) (width 0.8) (layer "B.Cu") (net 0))
 (segment (start 61.275 54.38) (end 63.095 54.38) (width 0.8) (layer "B.Cu") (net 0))
 (segment (start 58.975 51.435) (end 58.975 53.98) (width 0.4) (layer "B.Cu") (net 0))
 (segment (start 63.025 60.96) (end 63.025 63.34) (width 0.8) (layer "B.Cu") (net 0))
 (segment (start 58.975 49.37) (end 58.5 48.895) (width 0.4) (layer "B.Cu") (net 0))
 (segment (start 61.675 51.435) (end 61.775 51.435) (width 0.4) (layer "B.Cu") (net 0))
 (segment (start 58.975 51.435) (end 58.975 49.37) (width 0.4) (layer "B.Cu") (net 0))
 (segment (start 63.464213 52.525) (end 63.5 52.560787) (width 0.4) (layer "B.Cu") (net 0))
 (segment (start 56.04 63.34) (end 55.88 63.5) (width 0.8) (layer "B.Cu") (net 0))
 (segment (start 54.79 51.435) (end 55.88 52.525) (width 0.4) (layer "B.Cu") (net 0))
 (segment (start 59.055 51.355) (end 58.975 51.435) (width 0.4) (layer "B.Cu") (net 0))
 (segment (start 62.865 52.525) (end 63.464213 52.525) (width 0.4) (layer "B.Cu") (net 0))
 (segment (start 59.375 51.835) (end 58.975 51.435) (width 0.4) (layer "B.Cu") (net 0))
 (segment (start 61.775 51.435) (end 62.865 52.525) (width 0.4) (layer "B.Cu") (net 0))
 (segment (start 63.5 52.560787) (end 63.5 53.975) (width 0.4) (layer "B.Cu") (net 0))
 (segment (start 56.479213 52.525) (end 56.515 52.560787) (width 0.4) (layer "B.Cu") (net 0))
 (segment (start 60.325 60.96) (end 60.325 63.5) (width 0.8) (layer "B.Cu") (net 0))
 (segment (start 63.025 63.34) (end 62.865 63.5) (width 0.8) (layer "B.Cu") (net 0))
 (segment (start 54.69 51.435) (end 54.79 51.435) (width 0.4) (layer "B.Cu") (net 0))
 (segment (start 52.39 51.835) (end 51.99 51.435) (width 0.4) (layer "B.Cu") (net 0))
 (segment (start 51.99 51.435) (end 51.99 49.37) (width 0.4) (layer "B.Cu") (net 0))
 (segment (start 54.29 54.38) (end 56.11 54.38) (width 0.8) (layer "B.Cu") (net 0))
 (segment (start 60.325 57.38) (end 60.325 60.96) (width 0.8) (layer "B.Cu") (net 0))
 (segment (start 58.975 53.98) (end 59.375 54.38) (width 0.4) (layer "B.Cu") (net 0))
 (segment (start 52.07 51.355) (end 51.99 51.435) (width 0.4) (layer "B.Cu") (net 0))
 (segment (start 53.34 57.38) (end 53.34 60.96) (width 0.8) (layer "B.Cu") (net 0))
 (segment (start 55.88 52.525) (end 56.479213 52.525) (width 0.4) (layer "B.Cu") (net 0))
 (segment (start 56.515 52.560787) (end 56.515 53.975) (width 0.4) (layer "B.Cu") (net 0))
 (segment (start 56.04 60.96) (end 56.04 63.34) (width 0.8) (layer "B.Cu") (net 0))
 (segment (start 53.34 60.96) (end 53.34 63.5) (width 0.8) (layer "B.Cu") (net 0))
 (segment (start 56.11 54.38) (end 56.515 53.975) (width 0.8) (layer "B.Cu") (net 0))
 (segment (start 51.99 51.435) (end 51.99 53.98) (width 0.4) (layer "B.Cu") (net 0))
 (segment (start 63.095 54.38) (end 63.5 53.975) (width 0.8) (layer "B.Cu") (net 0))
 (segment (start 51.99 53.98) (end 52.39 54.38) (width 0.4) (layer "B.Cu") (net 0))
 (segment (start 51.99 49.37) (end 51.515 48.895) (width 0.4) (layer "B.Cu") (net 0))
 (segment (start 42.07 63.34) (end 41.91 63.5) (width 0.8) (layer "B.Cu") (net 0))
 (segment (start 38.02 49.37) (end 37.545 48.895) (width 0.4) (layer "B.Cu") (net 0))
 (segment (start 45.005 49.37) (end 44.53 48.895) (width 0.4) (layer "B.Cu") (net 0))
 (segment (start 48.895 52.525) (end 49.494213 52.525) (width 0.4) (layer "B.Cu") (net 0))
 (segment (start 49.494213 52.525) (end 49.53 52.560787) (width 0.4) (layer "B.Cu") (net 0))
 (segment (start 45.405 51.835) (end 45.005 51.435) (width 0.4) (layer "B.Cu") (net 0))
 (segment (start 38.1 51.355) (end 38.02 51.435) (width 0.4) (layer "B.Cu") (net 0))
 (segment (start 39.37 60.96) (end 39.37 63.5) (width 0.8) (layer "B.Cu") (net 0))
 (segment (start 38.02 51.435) (end 38.02 49.37) (width 0.4) (layer "B.Cu") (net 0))
 (segment (start 45.005 51.435) (end 45.005 53.98) (width 0.4) (layer "B.Cu") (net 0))
 (segment (start 38.42 51.835) (end 38.02 51.435) (width 0.4) (layer "B.Cu") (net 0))
 (segment (start 47.305 54.38) (end 49.125 54.38) (width 0.8) (layer "B.Cu") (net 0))
 (segment (start 41.91 52.525) (end 42.509213 52.525) (width 0.4) (layer "B.Cu") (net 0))
 (segment (start 40.72 51.435) (end 40.82 51.435) (width 0.4) (layer "B.Cu") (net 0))
 (segment (start 49.125 54.38) (end 49.53 53.975) (width 0.8) (layer "B.Cu") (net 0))
 (segment (start 38.02 51.435) (end 38.02 53.98) (width 0.4) (layer "B.Cu") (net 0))
 (segment (start 42.14 54.38) (end 42.545 53.975) (width 0.8) (layer "B.Cu") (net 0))
 (segment (start 45.005 51.435) (end 45.005 49.37) (width 0.4) (layer "B.Cu") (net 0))
 (segment (start 46.355 60.96) (end 46.355 63.5) (width 0.8) (layer "B.Cu") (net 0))
 (segment (start 42.509213 52.525) (end 42.545 52.560787) (width 0.4) (layer "B.Cu") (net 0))
 (segment (start 49.055 60.96) (end 49.055 63.34) (width 0.8) (layer "B.Cu") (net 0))
 (segment (start 49.055 63.34) (end 48.895 63.5) (width 0.8) (layer "B.Cu") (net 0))
 (segment (start 45.005 53.98) (end 45.405 54.38) (width 0.4) (layer "B.Cu") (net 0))
 (segment (start 42.07 60.96) (end 42.07 63.34) (width 0.8) (layer "B.Cu") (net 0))
 (segment (start 42.545 52.560787) (end 42.545 53.975) (width 0.4) (layer "B.Cu") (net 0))
 (segment (start 47.705 51.435) (end 47.805 51.435) (width 0.4) (layer "B.Cu") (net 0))
 (segment (start 38.02 53.98) (end 38.42 54.38) (width 0.4) (layer "B.Cu") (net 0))
 (segment (start 46.355 57.38) (end 46.355 60.96) (width 0.8) (layer "B.Cu") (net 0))
 (segment (start 40.82 51.435) (end 41.91 52.525) (width 0.4) (layer "B.Cu") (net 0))
 (segment (start 39.37 57.38) (end 39.37 60.96) (width 0.8) (layer "B.Cu") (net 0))
 (segment (start 47.805 51.435) (end 48.895 52.525) (width 0.4) (layer "B.Cu") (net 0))
 (segment (start 40.32 54.38) (end 42.14 54.38) (width 0.8) (layer "B.Cu") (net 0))
 (segment (start 49.53 52.560787) (end 49.53 53.975) (width 0.4) (layer "B.Cu") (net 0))
 (segment (start 45.085 51.355) (end 45.005 51.435) (width 0.4) (layer "B.Cu") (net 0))
 (segment (start 62.865 66.54) (end 62.865 64.135) (width 0.8) (layer "B.Cu") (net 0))
 (segment (start 75.745 51.435) (end 76.835 52.525) (width 0.4) (layer "B.Cu") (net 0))
 (segment (start 58.487919 45.085) (end 62.23 45.085) (width 0.4) (layer "B.Cu") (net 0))
 (segment (start 74.295 60.96) (end 74.295 63.5) (width 0.8) (layer "B.Cu") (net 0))
 (segment (start 75.245 54.38) (end 77.065 54.38) (width 0.8) (layer "B.Cu") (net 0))
 (segment (start 55.245 43.18) (end 55.245 48.34) (width 0.4) (layer "B.Cu") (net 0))
 (segment (start 77.065 54.38) (end 77.47 53.975) (width 0.8) (layer "B.Cu") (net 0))
 (segment (start 43.18 46.355) (end 41.83 47.705) (width 0.4) (layer "B.Cu") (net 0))
 (segment (start 62.865 66.54) (end 69.85 66.54) (width 0.8) (layer "B.Cu") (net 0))
 (segment (start 72.945 53.98) (end 73.345 54.38) (width 0.4) (layer "B.Cu") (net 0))
 (segment (start 69.85 66.54) (end 76.335 66.54) (width 0.8) (layer "B.Cu") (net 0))
 (segment (start 41.91 66.54) (end 41.91 64.135) (width 0.8) (layer "B.Cu") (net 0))
 (segment (start 46.99 46.355) (end 43.18 46.355) (width 0.4) (layer "B.Cu") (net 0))
 (segment (start 76.835 66.04) (end 76.835 64.135) (width 0.8) (layer "B.Cu") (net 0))
 (segment (start 74.295 57.38) (end 74.295 60.96) (width 0.8) (layer "B.Cu") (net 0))
 (segment (start 72.945 51.435) (end 72.945 49.37) (width 0.4) (layer "B.Cu") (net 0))
 (segment (start 60.325 43.18) (end 67.31 43.18) (width 0.4) (layer "B.Cu") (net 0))
 (segment (start 52.705 45.105) (end 51.455 46.355) (width 0.4) (layer "B.Cu") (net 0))
 (segment (start 33.655 66.54) (end 41.91 66.54) (width 0.8) (layer "B.Cu") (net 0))
 (segment (start 50.165 43.18) (end 46.99 46.355) (width 0.4) (layer "B.Cu") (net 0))
 (segment (start 73.345 51.835) (end 72.945 51.435) (width 0.4) (layer "B.Cu") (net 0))
 (segment (start 72.945 49.37) (end 72.47 48.895) (width 0.4) (layer "B.Cu") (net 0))
 (segment (start 55.88 66.54) (end 55.88 64.135) (width 0.8) (layer "B.Cu") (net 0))
 (segment (start 34.845 47.845) (end 34.845 48.895) (width 0.4) (layer "B.Cu") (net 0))
 (segment (start 48.895 66.54) (end 48.895 64.135) (width 0.8) (layer "B.Cu") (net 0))
 (segment (start 50.165 46.355) (end 48.815 47.705) (width 0.4) (layer "B.Cu") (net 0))
 (segment (start 41.83 47.705) (end 41.83 48.895) (width 0.4) (layer "B.Cu") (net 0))
 (segment (start 33.655 61.345) (end 34 61) (width 0.8) (layer "B.Cu") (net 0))
 (segment (start 41.91 66.54) (end 48.895 66.54) (width 0.8) (layer "B.Cu") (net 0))
 (segment (start 47.625 43.18) (end 39.51 43.18) (width 0.4) (layer "B.Cu") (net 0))
 (segment (start 77.434213 52.525) (end 77.47 52.560787) (width 0.4) (layer "B.Cu") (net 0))
 (segment (start 69.85 66.54) (end 69.85 64.135) (width 0.8) (layer "B.Cu") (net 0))
 (segment (start 77.47 52.560787) (end 77.47 53.975) (width 0.4) (layer "B.Cu") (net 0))
 (segment (start 57.785 44.382081) (end 58.487919 45.085) (width 0.4) (layer "B.Cu") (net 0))
 (segment (start 33.655 64) (end 33.655 61.345) (width 0.8) (layer "B.Cu") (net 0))
 (segment (start 76.835 52.525) (end 77.434213 52.525) (width 0.4) (layer "B.Cu") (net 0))
 (segment (start 48.895 66.54) (end 55.88 66.54) (width 0.8) (layer "B.Cu") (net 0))
 (segment (start 76.995 60.96) (end 76.995 63.34) (width 0.8) (layer "B.Cu") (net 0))
 (segment (start 67.31 43.18) (end 69.77 45.64) (width 0.4) (layer "B.Cu") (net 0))
 (segment (start 76.335 66.54) (end 76.835 66.04) (width 0.8) (layer "B.Cu") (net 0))
 (segment (start 62.785 45.64) (end 62.785 48.895) (width 0.4) (layer "B.Cu") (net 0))
 (segment (start 48.815 47.705) (end 48.815 48.895) (width 0.4) (layer "B.Cu") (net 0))
 (segment (start 51.455 46.355) (end 50.165 46.355) (width 0.4) (layer "B.Cu") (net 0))
 (segment (start 75.645 51.435) (end 75.745 51.435) (width 0.4) (layer "B.Cu") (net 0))
 (segment (start 55.245 48.34) (end 55.8 48.895) (width 0.4) (layer "B.Cu") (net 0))
 (segment (start 55.88 66.54) (end 62.865 66.54) (width 0.8) (layer "B.Cu") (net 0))
 (segment (start 57.785 43.18) (end 57.785 44.382081) (width 0.4) (layer "B.Cu") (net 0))
 (segment (start 52.705 43.18) (end 52.705 45.105) (width 0.4) (layer "B.Cu") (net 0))
 (segment (start 72.945 51.435) (end 72.945 53.98) (width 0.4) (layer "B.Cu") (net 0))
 (segment (start 76.995 63.34) (end 76.835 63.5) (width 0.8) (layer "B.Cu") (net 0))
 (segment (start 62.23 45.085) (end 62.785 45.64) (width 0.4) (layer "B.Cu") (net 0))
 (segment (start 73.025 51.355) (end 72.945 51.435) (width 0.4) (layer "B.Cu") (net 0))
 (segment (start 69.77 45.64) (end 69.77 48.895) (width 0.4) (layer "B.Cu") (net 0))
 (segment (start 39.51 43.18) (end 34.845 47.845) (width 0.4) (layer "B.Cu") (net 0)))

